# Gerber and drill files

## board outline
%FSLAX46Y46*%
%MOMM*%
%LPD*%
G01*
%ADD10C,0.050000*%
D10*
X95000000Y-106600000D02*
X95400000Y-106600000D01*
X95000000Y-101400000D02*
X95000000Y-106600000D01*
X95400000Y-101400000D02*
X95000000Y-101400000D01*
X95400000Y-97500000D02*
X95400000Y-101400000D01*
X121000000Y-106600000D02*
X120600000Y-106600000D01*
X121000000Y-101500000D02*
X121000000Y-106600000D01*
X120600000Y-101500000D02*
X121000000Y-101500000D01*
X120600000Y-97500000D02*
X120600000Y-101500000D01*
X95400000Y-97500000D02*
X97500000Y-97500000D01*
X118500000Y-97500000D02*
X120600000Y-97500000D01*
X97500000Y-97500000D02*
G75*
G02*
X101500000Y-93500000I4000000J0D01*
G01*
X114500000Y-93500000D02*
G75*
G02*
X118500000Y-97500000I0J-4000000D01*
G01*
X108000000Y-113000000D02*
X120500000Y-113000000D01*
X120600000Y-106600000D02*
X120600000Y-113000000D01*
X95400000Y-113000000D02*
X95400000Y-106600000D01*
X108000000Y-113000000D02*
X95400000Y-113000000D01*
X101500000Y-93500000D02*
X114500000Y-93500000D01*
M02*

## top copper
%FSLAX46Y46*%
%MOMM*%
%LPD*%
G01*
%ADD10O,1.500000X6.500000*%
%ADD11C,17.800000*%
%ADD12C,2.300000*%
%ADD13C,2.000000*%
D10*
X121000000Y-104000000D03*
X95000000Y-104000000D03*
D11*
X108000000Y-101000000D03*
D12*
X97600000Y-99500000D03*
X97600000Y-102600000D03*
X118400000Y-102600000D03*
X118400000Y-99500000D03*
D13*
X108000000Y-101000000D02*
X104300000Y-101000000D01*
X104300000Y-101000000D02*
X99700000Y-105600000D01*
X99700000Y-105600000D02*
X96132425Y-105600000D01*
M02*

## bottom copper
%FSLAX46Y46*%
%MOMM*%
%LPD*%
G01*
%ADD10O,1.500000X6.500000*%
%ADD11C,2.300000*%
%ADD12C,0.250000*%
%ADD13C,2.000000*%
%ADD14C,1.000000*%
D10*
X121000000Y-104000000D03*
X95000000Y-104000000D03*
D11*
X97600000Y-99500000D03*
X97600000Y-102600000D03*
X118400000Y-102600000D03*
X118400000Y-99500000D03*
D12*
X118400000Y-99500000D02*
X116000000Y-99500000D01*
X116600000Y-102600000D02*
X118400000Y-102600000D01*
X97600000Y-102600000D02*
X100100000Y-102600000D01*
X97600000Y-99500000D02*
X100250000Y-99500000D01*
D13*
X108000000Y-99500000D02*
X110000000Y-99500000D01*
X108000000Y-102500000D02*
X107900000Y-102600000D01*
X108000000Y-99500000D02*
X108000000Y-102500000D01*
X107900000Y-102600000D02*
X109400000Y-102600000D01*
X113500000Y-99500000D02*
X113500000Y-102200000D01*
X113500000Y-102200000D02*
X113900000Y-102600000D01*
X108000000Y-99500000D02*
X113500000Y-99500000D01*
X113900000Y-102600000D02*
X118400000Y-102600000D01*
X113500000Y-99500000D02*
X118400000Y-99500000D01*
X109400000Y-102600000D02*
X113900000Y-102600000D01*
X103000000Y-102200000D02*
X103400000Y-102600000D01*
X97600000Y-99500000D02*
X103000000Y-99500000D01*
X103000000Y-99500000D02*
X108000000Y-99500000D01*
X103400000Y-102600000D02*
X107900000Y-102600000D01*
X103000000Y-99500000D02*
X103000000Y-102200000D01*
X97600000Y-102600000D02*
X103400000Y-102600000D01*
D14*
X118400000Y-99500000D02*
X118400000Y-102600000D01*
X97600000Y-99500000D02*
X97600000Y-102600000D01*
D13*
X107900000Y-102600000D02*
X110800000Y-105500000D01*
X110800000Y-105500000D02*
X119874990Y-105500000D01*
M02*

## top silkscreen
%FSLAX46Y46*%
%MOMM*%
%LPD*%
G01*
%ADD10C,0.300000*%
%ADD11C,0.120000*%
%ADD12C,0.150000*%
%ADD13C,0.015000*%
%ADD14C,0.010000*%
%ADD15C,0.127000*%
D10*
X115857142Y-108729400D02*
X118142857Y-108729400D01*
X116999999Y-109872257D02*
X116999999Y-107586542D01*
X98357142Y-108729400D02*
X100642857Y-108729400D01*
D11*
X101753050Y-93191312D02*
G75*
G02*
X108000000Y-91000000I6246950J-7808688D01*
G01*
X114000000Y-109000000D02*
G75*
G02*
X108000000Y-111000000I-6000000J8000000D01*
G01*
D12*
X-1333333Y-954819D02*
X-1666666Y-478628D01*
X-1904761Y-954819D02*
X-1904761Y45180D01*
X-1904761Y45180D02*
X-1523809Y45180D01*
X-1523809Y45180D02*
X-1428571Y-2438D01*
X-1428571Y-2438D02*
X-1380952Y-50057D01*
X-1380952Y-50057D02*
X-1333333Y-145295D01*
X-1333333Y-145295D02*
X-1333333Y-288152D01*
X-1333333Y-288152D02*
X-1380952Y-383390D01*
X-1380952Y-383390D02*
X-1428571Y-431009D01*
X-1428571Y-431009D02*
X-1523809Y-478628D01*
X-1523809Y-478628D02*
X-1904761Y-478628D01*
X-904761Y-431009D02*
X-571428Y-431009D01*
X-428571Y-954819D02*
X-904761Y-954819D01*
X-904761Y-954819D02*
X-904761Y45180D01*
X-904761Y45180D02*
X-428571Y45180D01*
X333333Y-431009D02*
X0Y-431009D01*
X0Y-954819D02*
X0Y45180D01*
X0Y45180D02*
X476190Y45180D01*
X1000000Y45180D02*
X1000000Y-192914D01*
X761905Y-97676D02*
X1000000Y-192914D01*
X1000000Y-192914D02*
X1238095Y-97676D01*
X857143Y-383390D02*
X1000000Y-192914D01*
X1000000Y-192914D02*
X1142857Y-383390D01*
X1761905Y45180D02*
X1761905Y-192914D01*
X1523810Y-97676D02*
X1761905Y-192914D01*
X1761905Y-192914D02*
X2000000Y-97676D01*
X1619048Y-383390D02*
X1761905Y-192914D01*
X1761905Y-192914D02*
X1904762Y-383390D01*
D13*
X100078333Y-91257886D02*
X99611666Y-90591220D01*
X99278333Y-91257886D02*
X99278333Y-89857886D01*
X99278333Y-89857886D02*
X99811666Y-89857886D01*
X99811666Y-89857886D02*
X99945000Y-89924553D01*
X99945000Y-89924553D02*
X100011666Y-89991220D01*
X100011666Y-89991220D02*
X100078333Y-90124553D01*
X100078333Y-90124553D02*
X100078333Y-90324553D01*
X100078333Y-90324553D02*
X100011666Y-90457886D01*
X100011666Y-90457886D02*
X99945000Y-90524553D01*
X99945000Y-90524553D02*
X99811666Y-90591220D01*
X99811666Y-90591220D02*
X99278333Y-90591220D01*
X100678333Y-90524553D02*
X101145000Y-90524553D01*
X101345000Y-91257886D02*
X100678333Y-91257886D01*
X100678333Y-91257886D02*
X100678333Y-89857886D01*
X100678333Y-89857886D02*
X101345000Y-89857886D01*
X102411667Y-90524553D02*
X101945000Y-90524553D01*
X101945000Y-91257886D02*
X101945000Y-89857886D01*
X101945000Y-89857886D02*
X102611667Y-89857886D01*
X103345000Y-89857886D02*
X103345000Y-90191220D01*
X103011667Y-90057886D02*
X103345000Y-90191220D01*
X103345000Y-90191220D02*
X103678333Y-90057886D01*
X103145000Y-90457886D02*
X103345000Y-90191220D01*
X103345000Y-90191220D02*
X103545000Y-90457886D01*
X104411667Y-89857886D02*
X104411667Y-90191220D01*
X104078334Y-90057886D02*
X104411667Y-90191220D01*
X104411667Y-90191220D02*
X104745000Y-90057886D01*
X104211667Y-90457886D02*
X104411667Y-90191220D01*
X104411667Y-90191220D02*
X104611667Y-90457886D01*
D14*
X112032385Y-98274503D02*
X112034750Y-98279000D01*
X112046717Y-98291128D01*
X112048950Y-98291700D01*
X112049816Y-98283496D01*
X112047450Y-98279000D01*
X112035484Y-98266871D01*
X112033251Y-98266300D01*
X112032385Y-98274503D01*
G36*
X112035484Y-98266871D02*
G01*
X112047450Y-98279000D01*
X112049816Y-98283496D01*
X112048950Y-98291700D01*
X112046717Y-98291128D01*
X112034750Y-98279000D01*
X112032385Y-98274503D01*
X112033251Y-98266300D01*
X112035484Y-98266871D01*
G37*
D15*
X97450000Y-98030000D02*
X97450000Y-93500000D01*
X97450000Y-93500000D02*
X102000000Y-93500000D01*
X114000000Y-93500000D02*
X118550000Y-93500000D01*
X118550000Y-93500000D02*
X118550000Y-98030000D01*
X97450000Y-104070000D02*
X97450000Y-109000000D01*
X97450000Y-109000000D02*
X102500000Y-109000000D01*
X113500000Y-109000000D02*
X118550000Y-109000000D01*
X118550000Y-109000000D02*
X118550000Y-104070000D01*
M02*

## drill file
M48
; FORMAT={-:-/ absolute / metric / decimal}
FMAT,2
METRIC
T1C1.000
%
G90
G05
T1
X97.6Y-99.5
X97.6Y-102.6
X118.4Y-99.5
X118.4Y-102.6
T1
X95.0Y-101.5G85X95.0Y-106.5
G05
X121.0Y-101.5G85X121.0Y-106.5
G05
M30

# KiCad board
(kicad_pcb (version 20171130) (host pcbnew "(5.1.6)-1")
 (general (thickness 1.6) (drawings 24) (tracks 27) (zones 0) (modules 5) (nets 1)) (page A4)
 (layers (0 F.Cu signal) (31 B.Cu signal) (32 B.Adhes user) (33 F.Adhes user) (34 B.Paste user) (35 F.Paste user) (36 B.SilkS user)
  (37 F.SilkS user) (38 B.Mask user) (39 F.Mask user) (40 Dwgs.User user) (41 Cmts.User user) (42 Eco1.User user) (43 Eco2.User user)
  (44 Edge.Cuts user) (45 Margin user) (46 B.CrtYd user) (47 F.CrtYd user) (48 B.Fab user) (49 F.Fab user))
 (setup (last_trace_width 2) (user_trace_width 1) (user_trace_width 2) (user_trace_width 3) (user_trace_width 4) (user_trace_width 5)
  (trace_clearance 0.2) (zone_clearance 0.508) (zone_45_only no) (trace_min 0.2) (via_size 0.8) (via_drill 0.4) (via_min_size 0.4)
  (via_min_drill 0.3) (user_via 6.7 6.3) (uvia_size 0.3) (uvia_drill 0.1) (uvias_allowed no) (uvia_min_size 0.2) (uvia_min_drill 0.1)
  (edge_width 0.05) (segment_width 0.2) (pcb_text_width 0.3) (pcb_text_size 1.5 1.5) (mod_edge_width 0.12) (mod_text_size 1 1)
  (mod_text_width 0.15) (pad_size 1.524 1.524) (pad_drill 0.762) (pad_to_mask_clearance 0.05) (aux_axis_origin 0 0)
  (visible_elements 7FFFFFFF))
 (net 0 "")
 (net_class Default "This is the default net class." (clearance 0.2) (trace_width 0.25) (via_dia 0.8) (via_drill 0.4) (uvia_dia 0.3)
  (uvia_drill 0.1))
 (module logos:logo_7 (layer F.Cu) (at 113.4 100.2)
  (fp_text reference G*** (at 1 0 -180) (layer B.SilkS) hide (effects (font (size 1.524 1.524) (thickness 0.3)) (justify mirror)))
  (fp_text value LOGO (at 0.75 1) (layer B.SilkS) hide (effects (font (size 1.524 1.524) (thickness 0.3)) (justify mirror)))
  (fp_poly
   (pts (xy -1.367615 -1.925497) (xy -1.36525 -1.921) (xy -1.353283 -1.908872) (xy -1.35105 -1.9083) (xy -1.350184 -1.916504)
    (xy -1.35255 -1.921) (xy -1.364516 -1.933129) (xy -1.366749 -1.9337) (xy -1.367615 -1.925497))
   (layer F.SilkS) (width 0.01)))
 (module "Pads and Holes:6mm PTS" (layer F.Cu) (at 121 104)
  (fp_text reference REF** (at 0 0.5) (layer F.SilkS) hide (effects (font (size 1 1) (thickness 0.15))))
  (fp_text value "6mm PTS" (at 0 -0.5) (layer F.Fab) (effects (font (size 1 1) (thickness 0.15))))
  (pad 1 thru_hole oval (at 0 0) (size 1.5 6.5) (drill oval 1 6) (layers *.Cu *.Mask)))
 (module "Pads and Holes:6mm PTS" (layer F.Cu) (at 95 104)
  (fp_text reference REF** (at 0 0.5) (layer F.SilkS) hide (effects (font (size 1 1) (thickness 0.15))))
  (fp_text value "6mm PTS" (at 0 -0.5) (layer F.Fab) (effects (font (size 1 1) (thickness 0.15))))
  (pad 1 thru_hole oval (at 0 0) (size 1.5 6.5) (drill oval 1 6) (layers *.Cu *.Mask)))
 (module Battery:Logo (layer F.Cu) (at 0 0)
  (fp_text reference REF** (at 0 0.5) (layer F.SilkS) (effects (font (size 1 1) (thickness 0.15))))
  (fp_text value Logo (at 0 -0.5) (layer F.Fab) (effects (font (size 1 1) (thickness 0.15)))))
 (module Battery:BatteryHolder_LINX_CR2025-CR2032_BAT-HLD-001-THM (layer F.Cu) (at 108 101)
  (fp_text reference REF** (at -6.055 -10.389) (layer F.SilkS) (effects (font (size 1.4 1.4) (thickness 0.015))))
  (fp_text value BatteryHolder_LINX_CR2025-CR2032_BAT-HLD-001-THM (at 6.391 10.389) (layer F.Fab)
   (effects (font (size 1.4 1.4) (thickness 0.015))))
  (fp_line (start -10.55 -2.97) (end -10.55 -7.5) (layer F.SilkS) (width 0.127))
  (fp_line (start -10.55 -7.5) (end -6 -7.5) (layer F.SilkS) (width 0.127))
  (fp_line (start 6 -7.5) (end 10.55 -7.5) (layer F.SilkS) (width 0.127))
  (fp_line (start 10.55 -7.5) (end 10.55 -2.97) (layer F.SilkS) (width 0.127))
  (fp_line (start -10.55 3.07) (end -10.55 8) (layer F.SilkS) (width 0.127))
  (fp_line (start -10.55 8) (end -5.5 8) (layer F.SilkS) (width 0.127))
  (fp_line (start 5.5 8) (end 10.55 8) (layer F.SilkS) (width 0.127))
  (fp_line (start 10.55 8) (end 10.55 3.07) (layer F.SilkS) (width 0.127))
  (pad N smd circle (at 0 0) (size 17.8 17.8) (layers F.Cu F.Mask))
  (pad P1 thru_hole circle (at -10.4 -1.5) (size 2.3 2.3) (drill 1) (layers *.Cu *.Mask))
  (pad P2 thru_hole circle (at -10.4 1.6) (size 2.3 2.3) (drill 1) (layers *.Cu *.Mask))
  (pad P3 thru_hole circle (at 10.4 1.6) (size 2.3 2.3) (drill 1) (layers *.Cu *.Mask))
  (pad P4 thru_hole circle (at 10.4 -1.5) (size 2.3 2.3) (drill 1) (layers *.Cu *.Mask)))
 (gr_line (start 95 106.6) (end 95.4 106.6) (layer Edge.Cuts) (width 0.05))
 (gr_line (start 95 101.4) (end 95 106.6) (layer Edge.Cuts) (width 0.05))
 (gr_line (start 95.4 101.4) (end 95 101.4) (layer Edge.Cuts) (width 0.05))
 (gr_line (start 95.4 97.5) (end 95.4 101.4) (layer Edge.Cuts) (width 0.05))
 (gr_line (start 121 106.6) (end 120.6 106.6) (layer Edge.Cuts) (width 0.05))
 (gr_line (start 121 101.5) (end 121 106.6) (layer Edge.Cuts) (width 0.05))
 (gr_line (start 120.6 101.5) (end 121 101.5) (layer Edge.Cuts) (width 0.05))
 (gr_line (start 120.6 97.5) (end 120.6 101.5) (layer Edge.Cuts) (width 0.05))
 (gr_line (start 95.4 97.5) (end 97.5 97.5) (layer Edge.Cuts) (width 0.05))
 (gr_line (start 118.5 97.5) (end 120.6 97.5) (layer Edge.Cuts) (width 0.05))
 (gr_arc (start 101.5 97.5) (end 101.5 93.5) (angle -90) (layer Edge.Cuts) (width 0.05))
 (gr_arc (start 114.5 97.5) (end 118.5 97.5) (angle -90) (layer Edge.Cuts) (width 0.05))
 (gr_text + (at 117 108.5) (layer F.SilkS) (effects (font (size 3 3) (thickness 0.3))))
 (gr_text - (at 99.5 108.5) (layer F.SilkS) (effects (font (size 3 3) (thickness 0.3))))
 (gr_line (start 108 113) (end 120.5 113) (layer Edge.Cuts) (width 0.05))
 (gr_line (start 120.6 106.6) (end 120.6 113) (layer Edge.Cuts) (width 0.05))
 (gr_line (start 95.4 113) (end 95.4 106.6) (layer Edge.Cuts) (width 0.05))
 (gr_line (start 108 113) (end 95.4 113) (layer Edge.Cuts) (width 0.05))
 (gr_line (start 101.5 93.5) (end 114.5 93.5) (layer Edge.Cuts) (width 0.05))
 (gr_arc (start 108 101) (end 108 91) (angle -38.65980825) (layer F.SilkS) (width 0.12))
 (gr_arc (start 108 101) (end 108 111) (angle -36.86989765) (layer F.SilkS) (width 0.12))
 (segment (start 118.4 99.5) (end 116 99.5) (width 0.25) (layer B.Cu) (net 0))
 (segment (start 116.6 102.6) (end 118.4 102.6) (width 0.25) (layer B.Cu) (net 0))
 (segment (start 97.6 102.6) (end 100.1 102.6) (width 0.25) (layer B.Cu) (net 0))
 (segment (start 97.6 99.5) (end 100.25 99.5) (width 0.25) (layer B.Cu) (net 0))
 (segment (start 108 99.5) (end 110 99.5) (width 2) (layer B.Cu) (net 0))
 (segment (start 108 102.5) (end 107.9 102.6) (width 2) (layer B.Cu) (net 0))
 (segment (start 108 99.5) (end 108 102.5) (width 2) (layer B.Cu) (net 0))
 (segment (start 107.9 102.6) (end 109.4 102.6) (width 2) (layer B.Cu) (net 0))
 (segment (start 113.5 99.5) (end 113.5 102.2) (width 2) (layer B.Cu) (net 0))
 (segment (start 113.5 102.2) (end 113.9 102.6) (width 2) (layer B.Cu) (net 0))
 (segment (start 108 99.5) (end 113.5 99.5) (width 2) (layer B.Cu) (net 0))
 (segment (start 113.9 102.6) (end 118.4 102.6) (width 2) (layer B.Cu) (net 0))
 (segment (start 113.5 99.5) (end 118.4 99.5) (width 2) (layer B.Cu) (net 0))
 (segment (start 109.4 102.6) (end 113.9 102.6) (width 2) (layer B.Cu) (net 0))
 (segment (start 103 102.2) (end 103.4 102.6) (width 2) (layer B.Cu) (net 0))
 (segment (start 97.6 99.5) (end 103 99.5) (width 2) (layer B.Cu) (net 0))
 (segment (start 103 99.5) (end 108 99.5) (width 2) (layer B.Cu) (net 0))
 (segment (start 103.4 102.6) (end 107.9 102.6) (width 2) (layer B.Cu) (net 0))
 (segment (start 103 99.5) (end 103 102.2) (width 2) (layer B.Cu) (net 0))
 (segment (start 97.6 102.6) (end 103.4 102.6) (width 2) (layer B.Cu) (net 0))
 (segment (start 118.4 99.5) (end 118.4 102.6) (width 1) (layer B.Cu) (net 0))
 (segment (start 97.6 99.5) (end 97.6 102.6) (width 1) (layer B.Cu) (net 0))
 (segment (start 108 101) (end 104.3 101) (width 2) (layer F.Cu) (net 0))
 (segment (start 104.3 101) (end 99.7 105.6) (width 2) (layer F.Cu) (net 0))
 (segment (start 99.7 105.6) (end 96.132425 105.6) (width 2) (layer F.Cu) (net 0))
 (segment (start 107.9 102.6) (end 110.8 105.5) (width 2) (layer B.Cu) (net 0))
 (segment (start 110.8 105.5) (end 119.87499 105.5) (width 2) (layer B.Cu) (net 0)))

